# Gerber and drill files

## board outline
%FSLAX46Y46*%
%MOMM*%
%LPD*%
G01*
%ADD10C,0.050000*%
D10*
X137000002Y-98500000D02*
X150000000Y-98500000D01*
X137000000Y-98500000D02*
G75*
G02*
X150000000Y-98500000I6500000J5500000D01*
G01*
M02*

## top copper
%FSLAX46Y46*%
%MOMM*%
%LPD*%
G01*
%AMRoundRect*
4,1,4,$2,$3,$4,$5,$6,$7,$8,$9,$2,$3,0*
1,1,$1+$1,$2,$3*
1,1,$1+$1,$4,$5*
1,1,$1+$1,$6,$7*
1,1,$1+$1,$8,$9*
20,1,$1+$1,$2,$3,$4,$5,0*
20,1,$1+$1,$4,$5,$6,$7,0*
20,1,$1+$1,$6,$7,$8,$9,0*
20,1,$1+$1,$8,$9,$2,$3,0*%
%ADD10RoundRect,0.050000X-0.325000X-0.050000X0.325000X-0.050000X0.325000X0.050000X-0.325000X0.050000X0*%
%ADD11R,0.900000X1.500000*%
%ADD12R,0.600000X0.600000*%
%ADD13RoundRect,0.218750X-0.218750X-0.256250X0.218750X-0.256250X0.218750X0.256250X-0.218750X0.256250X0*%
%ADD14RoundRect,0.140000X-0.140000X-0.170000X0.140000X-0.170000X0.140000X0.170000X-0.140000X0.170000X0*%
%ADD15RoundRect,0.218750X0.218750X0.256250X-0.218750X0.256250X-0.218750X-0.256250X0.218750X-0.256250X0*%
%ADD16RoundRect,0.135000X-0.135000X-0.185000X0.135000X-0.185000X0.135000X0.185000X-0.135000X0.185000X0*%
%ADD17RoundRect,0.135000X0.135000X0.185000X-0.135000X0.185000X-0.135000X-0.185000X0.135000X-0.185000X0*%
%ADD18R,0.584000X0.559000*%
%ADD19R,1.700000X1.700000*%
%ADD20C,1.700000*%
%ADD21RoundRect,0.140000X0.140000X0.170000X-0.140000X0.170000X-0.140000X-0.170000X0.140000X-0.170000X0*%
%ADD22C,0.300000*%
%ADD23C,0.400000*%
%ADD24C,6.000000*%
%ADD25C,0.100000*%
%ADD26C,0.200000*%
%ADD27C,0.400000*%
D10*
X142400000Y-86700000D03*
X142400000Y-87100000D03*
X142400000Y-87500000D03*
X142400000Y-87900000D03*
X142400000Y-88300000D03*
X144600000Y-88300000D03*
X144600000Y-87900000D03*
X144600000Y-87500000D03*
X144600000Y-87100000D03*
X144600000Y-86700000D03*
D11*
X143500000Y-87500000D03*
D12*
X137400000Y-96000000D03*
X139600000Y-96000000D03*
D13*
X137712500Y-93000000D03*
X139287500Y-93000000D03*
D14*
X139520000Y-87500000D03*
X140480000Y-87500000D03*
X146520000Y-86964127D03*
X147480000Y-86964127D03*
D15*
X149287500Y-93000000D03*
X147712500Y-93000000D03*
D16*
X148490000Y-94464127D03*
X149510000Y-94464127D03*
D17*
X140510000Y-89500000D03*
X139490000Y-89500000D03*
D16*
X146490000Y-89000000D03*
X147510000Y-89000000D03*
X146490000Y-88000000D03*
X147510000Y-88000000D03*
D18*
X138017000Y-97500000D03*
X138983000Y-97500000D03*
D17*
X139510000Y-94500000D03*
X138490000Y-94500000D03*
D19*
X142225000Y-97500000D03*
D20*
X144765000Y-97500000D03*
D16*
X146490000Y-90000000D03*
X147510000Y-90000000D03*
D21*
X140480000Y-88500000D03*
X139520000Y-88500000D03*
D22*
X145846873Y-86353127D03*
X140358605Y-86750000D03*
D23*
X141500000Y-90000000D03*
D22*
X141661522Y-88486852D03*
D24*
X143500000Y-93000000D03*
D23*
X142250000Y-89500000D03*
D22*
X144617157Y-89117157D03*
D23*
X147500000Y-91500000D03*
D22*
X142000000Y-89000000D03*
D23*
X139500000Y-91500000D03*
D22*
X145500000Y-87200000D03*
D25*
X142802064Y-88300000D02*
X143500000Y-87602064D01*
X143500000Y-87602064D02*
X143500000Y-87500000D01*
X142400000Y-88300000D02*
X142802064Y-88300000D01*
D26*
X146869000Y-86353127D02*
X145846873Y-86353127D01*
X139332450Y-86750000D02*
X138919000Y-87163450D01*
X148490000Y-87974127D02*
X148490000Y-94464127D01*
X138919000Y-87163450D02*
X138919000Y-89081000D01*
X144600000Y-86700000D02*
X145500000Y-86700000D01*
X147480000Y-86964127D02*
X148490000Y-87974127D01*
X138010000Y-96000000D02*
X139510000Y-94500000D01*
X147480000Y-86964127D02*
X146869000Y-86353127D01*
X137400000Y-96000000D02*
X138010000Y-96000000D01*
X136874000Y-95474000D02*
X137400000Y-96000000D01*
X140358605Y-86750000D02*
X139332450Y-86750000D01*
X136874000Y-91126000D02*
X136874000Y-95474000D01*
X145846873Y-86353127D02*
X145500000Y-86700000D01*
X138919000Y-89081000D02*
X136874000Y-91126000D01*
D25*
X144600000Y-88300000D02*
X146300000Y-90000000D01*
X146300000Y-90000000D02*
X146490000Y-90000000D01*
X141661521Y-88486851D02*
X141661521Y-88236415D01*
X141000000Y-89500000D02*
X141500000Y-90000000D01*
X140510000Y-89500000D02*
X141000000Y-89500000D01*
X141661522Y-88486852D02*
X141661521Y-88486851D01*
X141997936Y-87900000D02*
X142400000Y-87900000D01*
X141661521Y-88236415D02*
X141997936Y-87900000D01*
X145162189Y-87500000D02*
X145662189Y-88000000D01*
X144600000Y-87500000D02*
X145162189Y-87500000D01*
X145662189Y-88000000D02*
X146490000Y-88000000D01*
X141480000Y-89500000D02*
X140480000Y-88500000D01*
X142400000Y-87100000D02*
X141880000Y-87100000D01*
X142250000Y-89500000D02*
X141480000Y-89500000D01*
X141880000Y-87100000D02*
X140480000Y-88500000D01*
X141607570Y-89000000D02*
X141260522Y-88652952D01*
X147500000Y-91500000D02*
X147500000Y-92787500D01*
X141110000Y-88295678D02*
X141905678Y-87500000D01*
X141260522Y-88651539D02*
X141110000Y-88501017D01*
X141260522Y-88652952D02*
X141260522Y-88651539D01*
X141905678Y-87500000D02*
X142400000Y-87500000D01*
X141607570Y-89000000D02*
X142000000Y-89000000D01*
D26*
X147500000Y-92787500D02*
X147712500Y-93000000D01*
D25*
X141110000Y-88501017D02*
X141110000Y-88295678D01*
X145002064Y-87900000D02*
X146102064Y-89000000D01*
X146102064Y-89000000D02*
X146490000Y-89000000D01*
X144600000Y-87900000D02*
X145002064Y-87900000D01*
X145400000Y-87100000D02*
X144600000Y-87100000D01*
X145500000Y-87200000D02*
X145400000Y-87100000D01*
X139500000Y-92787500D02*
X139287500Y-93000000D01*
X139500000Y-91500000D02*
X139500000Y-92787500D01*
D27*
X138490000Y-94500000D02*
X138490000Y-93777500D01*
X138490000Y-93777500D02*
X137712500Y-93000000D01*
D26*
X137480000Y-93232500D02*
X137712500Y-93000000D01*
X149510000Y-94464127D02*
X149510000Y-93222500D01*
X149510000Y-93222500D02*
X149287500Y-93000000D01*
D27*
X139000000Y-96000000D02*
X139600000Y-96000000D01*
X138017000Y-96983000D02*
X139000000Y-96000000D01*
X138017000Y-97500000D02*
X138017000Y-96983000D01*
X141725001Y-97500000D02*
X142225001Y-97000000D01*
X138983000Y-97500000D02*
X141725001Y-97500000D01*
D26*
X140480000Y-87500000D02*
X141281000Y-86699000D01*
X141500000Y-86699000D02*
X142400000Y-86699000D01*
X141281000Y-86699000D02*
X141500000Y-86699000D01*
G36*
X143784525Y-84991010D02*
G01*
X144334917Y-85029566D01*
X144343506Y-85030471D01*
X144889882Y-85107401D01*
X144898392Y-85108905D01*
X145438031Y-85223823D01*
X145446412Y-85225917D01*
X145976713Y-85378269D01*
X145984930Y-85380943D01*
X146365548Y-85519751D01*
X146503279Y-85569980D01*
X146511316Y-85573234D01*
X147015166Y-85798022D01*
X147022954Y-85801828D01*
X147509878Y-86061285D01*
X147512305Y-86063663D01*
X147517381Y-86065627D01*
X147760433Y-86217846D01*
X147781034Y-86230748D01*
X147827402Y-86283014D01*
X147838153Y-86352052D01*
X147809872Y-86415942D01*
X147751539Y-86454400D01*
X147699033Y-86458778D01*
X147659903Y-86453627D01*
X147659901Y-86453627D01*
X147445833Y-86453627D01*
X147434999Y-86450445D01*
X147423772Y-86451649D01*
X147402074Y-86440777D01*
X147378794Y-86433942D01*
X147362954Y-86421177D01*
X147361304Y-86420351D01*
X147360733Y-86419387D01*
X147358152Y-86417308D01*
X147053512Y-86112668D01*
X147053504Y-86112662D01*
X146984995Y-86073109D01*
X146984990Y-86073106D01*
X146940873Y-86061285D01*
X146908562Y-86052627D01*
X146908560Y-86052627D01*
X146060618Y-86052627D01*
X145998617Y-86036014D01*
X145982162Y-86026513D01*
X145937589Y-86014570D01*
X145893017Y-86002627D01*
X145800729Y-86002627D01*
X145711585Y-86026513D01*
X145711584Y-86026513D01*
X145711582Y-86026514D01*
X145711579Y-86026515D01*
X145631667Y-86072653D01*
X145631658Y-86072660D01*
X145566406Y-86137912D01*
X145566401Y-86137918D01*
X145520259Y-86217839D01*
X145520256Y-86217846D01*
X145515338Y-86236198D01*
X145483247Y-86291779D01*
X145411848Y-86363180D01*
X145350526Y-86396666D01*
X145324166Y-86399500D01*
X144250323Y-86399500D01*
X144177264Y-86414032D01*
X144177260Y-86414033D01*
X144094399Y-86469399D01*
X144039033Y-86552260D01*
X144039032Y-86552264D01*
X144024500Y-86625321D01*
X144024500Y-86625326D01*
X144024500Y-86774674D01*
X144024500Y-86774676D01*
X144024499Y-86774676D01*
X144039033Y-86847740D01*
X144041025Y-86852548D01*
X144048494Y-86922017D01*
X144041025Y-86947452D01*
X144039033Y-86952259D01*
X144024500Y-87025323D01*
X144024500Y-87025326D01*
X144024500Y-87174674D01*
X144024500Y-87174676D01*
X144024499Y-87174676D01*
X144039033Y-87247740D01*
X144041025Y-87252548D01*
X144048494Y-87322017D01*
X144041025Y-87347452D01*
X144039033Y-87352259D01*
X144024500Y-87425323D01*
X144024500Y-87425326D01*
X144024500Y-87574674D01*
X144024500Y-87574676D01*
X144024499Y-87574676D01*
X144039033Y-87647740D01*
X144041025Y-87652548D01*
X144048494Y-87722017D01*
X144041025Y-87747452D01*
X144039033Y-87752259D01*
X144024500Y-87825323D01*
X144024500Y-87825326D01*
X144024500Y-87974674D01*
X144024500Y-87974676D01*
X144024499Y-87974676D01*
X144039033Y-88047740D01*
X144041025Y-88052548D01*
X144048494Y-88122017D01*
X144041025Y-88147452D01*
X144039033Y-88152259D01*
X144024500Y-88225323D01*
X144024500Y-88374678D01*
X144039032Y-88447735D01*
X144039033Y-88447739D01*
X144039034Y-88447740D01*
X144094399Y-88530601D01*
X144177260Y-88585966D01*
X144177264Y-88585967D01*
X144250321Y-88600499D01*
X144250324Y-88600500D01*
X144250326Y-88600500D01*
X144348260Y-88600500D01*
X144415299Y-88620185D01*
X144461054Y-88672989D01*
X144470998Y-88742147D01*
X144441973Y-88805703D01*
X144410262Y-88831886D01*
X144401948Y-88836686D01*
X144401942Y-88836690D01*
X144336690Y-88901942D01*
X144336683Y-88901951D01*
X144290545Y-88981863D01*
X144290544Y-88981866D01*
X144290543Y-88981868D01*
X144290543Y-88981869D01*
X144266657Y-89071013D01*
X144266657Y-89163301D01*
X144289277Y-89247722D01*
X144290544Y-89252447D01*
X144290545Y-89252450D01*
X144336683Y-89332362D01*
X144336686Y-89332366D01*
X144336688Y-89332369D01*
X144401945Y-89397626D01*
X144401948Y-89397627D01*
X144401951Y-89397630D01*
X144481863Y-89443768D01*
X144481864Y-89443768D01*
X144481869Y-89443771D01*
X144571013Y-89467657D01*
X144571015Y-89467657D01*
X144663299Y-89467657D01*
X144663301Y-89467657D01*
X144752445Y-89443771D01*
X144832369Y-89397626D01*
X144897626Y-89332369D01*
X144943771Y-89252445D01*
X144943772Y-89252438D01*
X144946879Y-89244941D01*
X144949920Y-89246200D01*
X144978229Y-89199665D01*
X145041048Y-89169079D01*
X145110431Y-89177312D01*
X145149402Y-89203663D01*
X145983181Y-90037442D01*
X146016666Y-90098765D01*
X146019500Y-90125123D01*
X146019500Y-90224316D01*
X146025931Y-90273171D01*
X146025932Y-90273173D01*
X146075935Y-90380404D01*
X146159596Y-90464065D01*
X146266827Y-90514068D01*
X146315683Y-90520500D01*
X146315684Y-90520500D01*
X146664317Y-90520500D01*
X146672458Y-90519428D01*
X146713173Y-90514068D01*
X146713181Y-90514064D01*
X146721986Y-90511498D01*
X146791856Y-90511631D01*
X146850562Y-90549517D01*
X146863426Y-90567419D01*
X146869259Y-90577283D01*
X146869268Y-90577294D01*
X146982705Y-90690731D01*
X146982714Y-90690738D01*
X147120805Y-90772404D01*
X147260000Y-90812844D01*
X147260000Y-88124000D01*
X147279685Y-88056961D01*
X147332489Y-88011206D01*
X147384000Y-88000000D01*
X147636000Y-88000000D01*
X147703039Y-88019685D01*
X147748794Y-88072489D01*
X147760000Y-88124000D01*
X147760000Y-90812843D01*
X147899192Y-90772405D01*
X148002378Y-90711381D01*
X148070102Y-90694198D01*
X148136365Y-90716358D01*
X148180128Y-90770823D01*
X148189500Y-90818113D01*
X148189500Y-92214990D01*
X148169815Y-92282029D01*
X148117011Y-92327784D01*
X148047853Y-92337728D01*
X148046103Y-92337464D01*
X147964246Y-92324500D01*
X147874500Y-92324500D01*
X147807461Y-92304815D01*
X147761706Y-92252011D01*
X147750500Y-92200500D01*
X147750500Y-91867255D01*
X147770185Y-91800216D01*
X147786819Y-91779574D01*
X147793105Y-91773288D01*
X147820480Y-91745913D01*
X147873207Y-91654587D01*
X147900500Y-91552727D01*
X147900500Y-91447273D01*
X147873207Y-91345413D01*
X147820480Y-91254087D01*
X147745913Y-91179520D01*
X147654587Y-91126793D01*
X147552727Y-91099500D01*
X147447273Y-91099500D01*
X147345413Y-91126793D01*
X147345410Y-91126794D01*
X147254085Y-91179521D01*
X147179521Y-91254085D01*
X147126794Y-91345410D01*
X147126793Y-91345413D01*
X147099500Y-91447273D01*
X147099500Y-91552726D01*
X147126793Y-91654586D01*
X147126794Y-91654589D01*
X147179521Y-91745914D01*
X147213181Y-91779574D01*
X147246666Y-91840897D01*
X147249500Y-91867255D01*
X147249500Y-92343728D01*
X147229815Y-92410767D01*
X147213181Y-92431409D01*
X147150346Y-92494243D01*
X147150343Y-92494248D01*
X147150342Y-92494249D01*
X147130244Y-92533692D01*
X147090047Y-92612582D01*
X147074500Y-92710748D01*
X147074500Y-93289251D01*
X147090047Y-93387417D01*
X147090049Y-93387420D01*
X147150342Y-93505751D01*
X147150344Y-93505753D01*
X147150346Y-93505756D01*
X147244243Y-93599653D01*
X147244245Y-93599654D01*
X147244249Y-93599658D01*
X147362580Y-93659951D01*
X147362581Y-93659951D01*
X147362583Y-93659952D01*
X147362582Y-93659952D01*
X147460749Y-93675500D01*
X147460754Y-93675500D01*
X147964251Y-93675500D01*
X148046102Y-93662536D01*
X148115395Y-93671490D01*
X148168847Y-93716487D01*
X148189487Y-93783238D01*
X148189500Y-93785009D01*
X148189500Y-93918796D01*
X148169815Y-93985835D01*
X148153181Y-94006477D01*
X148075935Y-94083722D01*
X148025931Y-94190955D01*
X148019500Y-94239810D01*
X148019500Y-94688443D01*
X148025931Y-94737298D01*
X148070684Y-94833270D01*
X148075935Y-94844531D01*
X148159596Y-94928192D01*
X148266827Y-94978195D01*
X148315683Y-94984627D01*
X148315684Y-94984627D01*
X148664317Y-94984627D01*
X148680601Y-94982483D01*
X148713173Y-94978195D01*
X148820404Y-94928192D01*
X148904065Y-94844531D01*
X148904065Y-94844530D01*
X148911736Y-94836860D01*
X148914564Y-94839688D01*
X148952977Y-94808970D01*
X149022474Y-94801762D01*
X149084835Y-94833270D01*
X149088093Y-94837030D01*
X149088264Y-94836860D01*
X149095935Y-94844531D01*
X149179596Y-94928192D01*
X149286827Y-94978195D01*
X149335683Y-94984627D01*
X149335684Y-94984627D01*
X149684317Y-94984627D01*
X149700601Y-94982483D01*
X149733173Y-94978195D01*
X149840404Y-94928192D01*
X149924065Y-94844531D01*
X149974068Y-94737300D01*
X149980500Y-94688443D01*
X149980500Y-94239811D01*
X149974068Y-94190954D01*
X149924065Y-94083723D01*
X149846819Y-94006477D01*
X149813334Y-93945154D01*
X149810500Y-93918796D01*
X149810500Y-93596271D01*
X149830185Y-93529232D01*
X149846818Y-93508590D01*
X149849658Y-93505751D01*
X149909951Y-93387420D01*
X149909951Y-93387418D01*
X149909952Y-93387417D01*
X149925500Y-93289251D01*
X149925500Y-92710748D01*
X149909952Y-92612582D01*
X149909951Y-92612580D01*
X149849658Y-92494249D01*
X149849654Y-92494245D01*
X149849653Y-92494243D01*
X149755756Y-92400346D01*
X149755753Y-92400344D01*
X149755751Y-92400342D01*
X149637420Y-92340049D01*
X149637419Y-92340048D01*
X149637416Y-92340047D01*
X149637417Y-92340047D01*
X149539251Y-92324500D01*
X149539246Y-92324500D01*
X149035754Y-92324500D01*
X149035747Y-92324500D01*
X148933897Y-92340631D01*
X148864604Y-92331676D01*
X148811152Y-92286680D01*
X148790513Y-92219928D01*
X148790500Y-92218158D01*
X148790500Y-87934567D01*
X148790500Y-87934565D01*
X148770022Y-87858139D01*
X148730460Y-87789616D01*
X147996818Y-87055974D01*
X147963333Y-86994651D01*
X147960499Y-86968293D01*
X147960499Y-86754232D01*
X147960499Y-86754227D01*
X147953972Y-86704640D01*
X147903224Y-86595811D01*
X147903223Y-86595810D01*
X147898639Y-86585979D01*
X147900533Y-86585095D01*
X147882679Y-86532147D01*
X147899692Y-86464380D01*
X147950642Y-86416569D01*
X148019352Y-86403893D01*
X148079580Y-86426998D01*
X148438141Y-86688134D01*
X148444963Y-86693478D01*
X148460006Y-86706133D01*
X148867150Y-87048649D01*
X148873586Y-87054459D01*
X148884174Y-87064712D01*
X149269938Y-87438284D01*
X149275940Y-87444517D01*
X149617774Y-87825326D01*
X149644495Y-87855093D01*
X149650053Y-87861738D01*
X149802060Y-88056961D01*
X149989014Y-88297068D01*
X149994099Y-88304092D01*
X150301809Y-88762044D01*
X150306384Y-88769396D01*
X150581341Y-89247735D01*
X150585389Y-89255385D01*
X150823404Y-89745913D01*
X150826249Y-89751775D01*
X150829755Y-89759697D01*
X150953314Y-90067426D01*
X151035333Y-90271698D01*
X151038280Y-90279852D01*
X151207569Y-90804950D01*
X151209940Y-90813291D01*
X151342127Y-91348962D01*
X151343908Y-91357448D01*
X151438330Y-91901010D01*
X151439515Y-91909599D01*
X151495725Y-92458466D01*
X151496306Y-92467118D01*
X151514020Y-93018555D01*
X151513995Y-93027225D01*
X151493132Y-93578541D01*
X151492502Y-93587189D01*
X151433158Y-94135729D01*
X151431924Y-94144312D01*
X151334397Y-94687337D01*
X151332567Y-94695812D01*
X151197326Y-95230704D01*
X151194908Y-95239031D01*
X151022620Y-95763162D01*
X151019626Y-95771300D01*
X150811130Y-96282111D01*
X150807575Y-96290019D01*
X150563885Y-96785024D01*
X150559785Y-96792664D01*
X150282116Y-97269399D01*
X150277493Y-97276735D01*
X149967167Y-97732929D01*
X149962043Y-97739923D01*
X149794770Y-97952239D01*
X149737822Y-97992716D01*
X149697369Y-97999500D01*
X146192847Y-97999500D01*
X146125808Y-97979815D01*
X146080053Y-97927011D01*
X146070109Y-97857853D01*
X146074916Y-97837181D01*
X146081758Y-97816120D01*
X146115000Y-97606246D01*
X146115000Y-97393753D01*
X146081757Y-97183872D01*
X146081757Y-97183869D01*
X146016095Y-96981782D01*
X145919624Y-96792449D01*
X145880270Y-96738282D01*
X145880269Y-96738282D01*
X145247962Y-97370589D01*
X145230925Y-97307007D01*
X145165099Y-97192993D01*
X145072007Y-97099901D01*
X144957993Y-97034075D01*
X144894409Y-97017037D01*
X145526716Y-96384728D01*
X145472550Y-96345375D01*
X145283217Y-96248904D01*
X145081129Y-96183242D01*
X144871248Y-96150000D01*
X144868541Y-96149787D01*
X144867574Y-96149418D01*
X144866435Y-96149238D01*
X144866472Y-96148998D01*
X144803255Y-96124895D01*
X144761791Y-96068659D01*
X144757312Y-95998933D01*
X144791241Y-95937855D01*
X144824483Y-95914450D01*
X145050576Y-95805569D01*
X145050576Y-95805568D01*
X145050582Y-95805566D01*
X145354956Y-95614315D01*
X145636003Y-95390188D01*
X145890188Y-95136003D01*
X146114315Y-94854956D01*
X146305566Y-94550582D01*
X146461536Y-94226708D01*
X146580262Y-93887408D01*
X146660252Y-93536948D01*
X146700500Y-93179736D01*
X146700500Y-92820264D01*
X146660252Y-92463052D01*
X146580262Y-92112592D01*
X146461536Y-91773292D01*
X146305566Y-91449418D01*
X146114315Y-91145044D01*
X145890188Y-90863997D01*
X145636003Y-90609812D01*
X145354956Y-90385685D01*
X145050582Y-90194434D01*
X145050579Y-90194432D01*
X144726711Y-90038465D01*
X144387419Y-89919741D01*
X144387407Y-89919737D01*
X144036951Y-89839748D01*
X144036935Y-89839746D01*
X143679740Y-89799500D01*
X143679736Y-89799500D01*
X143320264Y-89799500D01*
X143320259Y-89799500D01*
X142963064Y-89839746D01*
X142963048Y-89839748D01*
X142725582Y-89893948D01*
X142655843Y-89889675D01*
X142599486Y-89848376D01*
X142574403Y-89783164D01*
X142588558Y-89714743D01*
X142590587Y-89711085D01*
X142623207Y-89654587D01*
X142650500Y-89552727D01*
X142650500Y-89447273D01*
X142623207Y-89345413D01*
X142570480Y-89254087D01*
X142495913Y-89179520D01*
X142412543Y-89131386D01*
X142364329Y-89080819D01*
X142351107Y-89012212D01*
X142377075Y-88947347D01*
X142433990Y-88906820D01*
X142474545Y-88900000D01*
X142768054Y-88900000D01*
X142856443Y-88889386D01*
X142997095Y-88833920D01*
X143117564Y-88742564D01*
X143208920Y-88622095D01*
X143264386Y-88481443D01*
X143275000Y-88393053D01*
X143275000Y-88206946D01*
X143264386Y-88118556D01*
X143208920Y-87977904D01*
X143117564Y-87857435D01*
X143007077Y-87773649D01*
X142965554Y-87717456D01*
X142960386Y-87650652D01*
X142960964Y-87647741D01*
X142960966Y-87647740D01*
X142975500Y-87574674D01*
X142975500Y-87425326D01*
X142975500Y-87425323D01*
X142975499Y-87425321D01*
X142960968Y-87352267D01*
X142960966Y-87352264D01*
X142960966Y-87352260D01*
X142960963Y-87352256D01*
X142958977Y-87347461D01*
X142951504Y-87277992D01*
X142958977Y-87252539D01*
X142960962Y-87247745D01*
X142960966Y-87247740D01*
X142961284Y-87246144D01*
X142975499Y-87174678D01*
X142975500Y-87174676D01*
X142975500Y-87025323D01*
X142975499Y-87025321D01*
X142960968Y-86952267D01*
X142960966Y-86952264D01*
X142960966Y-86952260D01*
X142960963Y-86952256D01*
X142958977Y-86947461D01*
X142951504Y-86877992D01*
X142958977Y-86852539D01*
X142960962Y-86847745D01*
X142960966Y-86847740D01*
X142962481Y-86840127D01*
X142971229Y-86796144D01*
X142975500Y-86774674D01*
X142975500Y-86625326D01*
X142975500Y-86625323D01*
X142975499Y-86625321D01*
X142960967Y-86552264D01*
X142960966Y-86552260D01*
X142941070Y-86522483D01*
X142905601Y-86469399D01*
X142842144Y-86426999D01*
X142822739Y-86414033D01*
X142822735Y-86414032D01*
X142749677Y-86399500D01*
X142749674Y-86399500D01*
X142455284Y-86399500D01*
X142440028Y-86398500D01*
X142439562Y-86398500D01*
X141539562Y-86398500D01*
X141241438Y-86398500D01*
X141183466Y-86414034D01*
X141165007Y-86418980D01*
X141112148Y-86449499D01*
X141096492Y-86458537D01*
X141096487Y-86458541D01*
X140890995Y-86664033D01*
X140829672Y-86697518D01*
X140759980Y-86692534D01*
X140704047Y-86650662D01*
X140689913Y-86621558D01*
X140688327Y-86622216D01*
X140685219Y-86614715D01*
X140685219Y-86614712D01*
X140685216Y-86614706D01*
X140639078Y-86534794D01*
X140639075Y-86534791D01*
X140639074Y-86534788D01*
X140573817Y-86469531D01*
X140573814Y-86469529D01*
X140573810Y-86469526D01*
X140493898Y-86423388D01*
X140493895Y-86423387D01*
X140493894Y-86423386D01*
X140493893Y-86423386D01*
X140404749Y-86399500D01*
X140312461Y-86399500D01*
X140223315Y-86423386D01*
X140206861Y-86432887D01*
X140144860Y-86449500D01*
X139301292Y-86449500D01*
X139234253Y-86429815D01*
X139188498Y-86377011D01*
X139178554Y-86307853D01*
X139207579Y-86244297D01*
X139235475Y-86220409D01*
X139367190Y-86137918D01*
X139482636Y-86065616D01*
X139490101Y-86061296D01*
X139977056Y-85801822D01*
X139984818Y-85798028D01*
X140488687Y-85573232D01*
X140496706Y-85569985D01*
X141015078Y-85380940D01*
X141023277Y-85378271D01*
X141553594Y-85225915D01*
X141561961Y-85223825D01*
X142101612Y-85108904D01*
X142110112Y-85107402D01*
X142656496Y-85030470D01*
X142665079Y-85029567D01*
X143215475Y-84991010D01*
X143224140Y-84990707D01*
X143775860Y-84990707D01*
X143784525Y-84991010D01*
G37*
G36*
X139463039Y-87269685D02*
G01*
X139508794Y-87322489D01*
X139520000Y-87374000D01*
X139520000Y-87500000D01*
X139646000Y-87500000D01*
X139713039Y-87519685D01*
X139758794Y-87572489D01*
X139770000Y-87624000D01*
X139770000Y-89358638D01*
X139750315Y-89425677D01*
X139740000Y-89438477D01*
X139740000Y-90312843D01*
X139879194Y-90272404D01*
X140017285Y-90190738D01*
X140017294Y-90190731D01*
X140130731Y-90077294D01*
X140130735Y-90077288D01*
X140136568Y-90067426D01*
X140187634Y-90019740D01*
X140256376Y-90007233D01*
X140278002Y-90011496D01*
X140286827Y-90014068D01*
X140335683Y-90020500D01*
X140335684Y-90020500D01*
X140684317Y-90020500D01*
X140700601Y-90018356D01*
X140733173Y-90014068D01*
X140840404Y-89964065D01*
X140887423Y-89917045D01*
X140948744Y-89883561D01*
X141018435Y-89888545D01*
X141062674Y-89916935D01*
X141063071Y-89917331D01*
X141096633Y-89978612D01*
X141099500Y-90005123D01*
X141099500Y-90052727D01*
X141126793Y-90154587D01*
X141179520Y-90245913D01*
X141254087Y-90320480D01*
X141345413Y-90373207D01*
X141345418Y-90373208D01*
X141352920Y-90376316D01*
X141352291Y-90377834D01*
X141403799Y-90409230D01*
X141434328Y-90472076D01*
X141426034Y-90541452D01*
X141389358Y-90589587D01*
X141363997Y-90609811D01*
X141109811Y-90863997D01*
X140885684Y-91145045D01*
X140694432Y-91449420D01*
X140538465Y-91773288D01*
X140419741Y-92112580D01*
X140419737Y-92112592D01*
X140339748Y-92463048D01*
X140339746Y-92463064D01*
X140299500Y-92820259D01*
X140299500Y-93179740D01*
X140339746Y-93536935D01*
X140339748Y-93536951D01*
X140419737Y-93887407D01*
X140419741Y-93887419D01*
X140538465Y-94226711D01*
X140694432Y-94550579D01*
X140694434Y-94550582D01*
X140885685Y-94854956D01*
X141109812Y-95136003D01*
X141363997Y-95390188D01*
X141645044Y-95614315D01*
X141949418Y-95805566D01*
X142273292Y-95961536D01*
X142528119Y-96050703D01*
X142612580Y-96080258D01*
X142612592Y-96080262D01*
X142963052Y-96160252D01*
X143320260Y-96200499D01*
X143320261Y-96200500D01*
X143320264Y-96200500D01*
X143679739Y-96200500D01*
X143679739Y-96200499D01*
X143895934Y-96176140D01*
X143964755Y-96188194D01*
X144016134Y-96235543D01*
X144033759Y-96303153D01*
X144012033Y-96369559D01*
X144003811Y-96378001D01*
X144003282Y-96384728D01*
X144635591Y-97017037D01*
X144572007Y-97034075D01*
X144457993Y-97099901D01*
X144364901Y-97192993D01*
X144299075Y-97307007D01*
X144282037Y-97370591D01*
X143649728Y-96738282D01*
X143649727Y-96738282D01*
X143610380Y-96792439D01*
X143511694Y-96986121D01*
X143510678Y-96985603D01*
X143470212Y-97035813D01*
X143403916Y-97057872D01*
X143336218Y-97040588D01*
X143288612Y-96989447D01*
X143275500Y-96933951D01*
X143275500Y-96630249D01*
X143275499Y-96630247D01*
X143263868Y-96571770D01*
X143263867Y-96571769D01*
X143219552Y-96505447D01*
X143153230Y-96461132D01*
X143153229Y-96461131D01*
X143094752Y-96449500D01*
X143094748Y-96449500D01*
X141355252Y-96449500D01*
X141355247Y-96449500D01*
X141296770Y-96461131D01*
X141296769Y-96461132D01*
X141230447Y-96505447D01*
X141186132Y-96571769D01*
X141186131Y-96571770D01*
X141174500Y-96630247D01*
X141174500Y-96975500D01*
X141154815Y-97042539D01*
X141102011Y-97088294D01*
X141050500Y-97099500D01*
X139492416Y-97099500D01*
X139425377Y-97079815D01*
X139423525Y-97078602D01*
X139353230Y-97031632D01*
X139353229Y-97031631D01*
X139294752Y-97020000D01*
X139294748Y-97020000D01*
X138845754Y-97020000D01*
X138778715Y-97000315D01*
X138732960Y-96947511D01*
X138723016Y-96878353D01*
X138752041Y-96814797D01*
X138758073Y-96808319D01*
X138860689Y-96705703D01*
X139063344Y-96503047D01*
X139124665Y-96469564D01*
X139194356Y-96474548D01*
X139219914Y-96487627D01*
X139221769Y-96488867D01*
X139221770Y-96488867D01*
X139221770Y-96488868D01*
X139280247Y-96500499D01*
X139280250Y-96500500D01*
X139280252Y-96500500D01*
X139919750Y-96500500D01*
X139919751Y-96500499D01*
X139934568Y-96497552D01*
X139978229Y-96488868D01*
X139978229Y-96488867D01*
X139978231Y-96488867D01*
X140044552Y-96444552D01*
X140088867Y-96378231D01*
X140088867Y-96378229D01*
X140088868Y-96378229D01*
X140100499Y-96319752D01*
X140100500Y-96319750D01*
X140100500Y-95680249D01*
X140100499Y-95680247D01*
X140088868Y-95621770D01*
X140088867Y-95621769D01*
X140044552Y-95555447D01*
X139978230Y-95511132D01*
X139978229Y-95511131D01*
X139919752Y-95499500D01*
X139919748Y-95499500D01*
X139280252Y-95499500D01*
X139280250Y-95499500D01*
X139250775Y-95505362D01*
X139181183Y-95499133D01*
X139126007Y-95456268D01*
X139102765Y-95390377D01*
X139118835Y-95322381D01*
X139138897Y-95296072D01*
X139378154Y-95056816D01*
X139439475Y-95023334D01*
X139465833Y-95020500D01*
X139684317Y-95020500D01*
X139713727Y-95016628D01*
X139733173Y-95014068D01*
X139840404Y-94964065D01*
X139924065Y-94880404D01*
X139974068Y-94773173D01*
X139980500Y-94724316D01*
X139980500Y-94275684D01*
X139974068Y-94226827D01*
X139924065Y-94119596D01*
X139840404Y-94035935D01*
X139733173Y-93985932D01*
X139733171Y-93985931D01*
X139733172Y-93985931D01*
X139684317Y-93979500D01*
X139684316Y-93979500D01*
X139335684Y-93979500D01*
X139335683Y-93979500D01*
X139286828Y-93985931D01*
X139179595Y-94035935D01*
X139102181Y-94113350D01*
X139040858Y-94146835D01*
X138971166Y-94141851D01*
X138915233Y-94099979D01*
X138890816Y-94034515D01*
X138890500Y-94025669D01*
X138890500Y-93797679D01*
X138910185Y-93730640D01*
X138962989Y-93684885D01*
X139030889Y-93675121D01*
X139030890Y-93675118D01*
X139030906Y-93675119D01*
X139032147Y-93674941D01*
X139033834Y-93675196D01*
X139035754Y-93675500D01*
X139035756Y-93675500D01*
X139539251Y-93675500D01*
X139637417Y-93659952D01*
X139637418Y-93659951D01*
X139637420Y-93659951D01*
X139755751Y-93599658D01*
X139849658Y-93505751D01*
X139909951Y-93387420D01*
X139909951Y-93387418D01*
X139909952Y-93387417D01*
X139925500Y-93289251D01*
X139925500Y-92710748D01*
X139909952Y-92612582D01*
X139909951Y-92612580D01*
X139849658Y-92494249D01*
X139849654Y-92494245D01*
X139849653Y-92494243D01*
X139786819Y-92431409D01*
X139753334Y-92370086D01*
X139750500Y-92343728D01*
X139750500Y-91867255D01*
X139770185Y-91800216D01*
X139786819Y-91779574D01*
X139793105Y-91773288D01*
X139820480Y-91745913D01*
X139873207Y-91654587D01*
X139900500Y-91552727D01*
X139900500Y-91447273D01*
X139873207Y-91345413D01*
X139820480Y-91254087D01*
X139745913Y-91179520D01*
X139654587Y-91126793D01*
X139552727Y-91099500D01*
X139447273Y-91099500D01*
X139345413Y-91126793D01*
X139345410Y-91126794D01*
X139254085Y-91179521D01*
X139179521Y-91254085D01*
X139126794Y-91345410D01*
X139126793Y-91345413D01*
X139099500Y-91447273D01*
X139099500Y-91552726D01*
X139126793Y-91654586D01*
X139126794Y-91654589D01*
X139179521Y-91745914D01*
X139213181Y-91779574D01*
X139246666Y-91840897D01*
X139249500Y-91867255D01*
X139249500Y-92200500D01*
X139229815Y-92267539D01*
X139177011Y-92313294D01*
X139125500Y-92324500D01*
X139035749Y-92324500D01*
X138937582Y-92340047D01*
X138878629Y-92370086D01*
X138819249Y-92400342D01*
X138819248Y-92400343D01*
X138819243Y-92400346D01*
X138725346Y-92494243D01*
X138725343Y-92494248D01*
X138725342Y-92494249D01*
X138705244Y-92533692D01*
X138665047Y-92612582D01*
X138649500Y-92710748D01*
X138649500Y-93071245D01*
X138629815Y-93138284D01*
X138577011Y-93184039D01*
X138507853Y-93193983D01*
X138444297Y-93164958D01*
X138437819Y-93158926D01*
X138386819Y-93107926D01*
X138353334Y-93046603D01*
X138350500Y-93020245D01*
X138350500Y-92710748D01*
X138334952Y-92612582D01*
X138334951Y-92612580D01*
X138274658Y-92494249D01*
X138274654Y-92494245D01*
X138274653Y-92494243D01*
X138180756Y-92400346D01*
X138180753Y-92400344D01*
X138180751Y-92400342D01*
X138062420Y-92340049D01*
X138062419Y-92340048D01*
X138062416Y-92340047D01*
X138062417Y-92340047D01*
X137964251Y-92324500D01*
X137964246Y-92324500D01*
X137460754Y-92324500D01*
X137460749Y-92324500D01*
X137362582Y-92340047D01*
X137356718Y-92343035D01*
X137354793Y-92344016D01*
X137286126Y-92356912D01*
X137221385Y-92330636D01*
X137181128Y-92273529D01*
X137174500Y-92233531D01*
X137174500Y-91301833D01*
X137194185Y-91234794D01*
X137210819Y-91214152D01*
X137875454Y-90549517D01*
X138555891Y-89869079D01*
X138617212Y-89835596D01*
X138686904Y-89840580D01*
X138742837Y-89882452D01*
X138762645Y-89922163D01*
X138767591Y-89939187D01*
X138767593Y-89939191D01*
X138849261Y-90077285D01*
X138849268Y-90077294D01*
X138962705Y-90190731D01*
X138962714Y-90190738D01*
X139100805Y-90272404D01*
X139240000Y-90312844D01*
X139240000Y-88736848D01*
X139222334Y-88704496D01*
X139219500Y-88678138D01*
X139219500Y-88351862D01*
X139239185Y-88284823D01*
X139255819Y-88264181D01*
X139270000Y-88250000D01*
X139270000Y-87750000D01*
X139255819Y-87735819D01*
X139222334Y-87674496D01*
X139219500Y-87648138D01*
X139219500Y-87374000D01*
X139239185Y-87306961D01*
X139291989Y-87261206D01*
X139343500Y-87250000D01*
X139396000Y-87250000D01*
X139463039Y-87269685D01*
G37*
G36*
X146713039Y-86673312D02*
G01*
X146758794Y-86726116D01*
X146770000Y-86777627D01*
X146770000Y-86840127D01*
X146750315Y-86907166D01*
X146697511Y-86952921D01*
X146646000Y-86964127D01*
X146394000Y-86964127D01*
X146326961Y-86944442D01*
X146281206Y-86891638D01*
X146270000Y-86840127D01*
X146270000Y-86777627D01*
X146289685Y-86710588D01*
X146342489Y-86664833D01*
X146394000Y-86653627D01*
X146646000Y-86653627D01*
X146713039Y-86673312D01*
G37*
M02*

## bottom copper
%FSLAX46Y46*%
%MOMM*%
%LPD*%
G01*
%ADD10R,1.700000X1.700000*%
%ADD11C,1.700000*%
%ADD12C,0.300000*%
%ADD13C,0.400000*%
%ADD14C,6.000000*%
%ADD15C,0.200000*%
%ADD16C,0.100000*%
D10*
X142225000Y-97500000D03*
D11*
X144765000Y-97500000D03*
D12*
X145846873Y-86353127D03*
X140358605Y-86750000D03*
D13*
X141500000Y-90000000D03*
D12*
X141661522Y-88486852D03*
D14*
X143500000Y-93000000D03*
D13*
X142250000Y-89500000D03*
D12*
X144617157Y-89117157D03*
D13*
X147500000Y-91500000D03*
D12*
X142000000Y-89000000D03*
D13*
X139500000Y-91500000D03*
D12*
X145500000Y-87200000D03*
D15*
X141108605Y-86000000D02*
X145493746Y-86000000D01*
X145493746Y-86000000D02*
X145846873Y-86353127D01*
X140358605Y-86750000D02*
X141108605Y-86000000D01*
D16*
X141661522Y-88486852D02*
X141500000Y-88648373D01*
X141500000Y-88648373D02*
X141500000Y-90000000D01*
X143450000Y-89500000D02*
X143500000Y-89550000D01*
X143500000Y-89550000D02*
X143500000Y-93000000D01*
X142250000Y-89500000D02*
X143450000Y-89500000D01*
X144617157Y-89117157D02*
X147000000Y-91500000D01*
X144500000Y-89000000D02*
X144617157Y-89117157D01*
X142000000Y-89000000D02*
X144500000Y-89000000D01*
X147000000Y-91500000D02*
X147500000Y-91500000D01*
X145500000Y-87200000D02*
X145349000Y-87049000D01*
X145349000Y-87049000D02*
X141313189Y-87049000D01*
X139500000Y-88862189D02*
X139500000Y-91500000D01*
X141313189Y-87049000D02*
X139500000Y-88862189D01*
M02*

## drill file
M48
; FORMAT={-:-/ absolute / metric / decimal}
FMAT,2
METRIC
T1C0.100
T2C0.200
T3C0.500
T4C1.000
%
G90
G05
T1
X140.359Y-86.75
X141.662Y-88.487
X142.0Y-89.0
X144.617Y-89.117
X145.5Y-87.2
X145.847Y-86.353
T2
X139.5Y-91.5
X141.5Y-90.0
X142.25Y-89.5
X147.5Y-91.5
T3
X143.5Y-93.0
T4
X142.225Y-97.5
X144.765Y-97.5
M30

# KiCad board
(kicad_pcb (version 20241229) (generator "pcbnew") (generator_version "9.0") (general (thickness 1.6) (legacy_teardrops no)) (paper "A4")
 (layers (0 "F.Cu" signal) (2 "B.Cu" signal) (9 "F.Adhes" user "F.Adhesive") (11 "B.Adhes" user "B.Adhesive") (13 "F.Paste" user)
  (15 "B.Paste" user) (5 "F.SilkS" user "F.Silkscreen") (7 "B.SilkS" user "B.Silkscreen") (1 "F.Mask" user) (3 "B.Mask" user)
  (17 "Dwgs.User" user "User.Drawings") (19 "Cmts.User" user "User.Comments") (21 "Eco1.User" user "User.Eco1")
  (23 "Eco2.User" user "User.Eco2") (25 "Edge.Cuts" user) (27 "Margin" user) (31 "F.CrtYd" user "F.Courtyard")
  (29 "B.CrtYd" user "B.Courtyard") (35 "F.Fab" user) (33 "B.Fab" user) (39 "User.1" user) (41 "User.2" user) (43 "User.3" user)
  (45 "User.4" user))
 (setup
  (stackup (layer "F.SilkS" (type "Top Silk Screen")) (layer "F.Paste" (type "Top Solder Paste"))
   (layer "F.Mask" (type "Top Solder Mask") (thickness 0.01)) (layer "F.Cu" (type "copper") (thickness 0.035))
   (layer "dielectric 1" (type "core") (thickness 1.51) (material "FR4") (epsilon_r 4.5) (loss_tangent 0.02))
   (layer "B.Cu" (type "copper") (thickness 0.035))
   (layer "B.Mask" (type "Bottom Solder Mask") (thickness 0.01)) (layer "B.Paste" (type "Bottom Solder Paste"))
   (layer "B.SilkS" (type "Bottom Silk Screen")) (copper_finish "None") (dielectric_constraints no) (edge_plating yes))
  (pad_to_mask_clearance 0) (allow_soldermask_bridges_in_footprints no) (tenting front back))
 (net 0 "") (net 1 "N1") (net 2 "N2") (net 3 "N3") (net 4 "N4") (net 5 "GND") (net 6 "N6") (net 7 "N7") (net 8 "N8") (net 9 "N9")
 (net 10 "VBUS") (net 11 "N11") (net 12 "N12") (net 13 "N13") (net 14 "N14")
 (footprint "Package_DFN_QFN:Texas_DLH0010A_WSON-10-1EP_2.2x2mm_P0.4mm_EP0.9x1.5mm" (layer "F.Cu") (at 143.5 87.5)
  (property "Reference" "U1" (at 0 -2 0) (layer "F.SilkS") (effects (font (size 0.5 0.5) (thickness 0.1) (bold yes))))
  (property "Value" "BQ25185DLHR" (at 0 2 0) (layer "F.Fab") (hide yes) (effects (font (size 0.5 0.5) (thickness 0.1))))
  (pad "" smd roundrect (at 0 0) (size 0.84 1.41) (layers "F.Paste") (roundrect_rratio 0.25))
  (pad "1" smd roundrect (at -1.1 -0.8) (size 0.75 0.2) (layers "F.Cu" "F.Mask" "F.Paste") (roundrect_rratio 0.25) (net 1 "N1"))
  (pad "2" smd roundrect (at -1.1 -0.4) (size 0.75 0.2) (layers "F.Cu" "F.Mask" "F.Paste") (roundrect_rratio 0.25) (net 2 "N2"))
  (pad "3" smd roundrect (at -1.1 0) (size 0.75 0.2) (layers "F.Cu" "F.Mask" "F.Paste") (roundrect_rratio 0.25) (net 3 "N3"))
  (pad "4" smd roundrect (at -1.1 0.4) (size 0.75 0.2) (layers "F.Cu" "F.Mask" "F.Paste") (roundrect_rratio 0.25) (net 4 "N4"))
  (pad "5" smd roundrect (at -1.1 0.8) (size 0.75 0.2) (layers "F.Cu" "F.Mask" "F.Paste") (roundrect_rratio 0.25) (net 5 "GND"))
  (pad "6" smd roundrect (at 1.1 0.8) (size 0.75 0.2) (layers "F.Cu" "F.Mask" "F.Paste") (roundrect_rratio 0.25) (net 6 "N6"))
  (pad "7" smd roundrect (at 1.1 0.4) (size 0.75 0.2) (layers "F.Cu" "F.Mask" "F.Paste") (roundrect_rratio 0.25) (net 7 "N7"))
  (pad "8" smd roundrect (at 1.1 0) (size 0.75 0.2) (layers "F.Cu" "F.Mask" "F.Paste") (roundrect_rratio 0.25) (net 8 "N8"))
  (pad "9" smd roundrect (at 1.1 -0.4) (size 0.75 0.2) (layers "F.Cu" "F.Mask" "F.Paste") (roundrect_rratio 0.25) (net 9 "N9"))
  (pad "10" smd roundrect (at 1.1 -0.8) (size 0.75 0.2) (layers "F.Cu" "F.Mask" "F.Paste") (roundrect_rratio 0.25) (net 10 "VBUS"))
  (pad "11" smd rect (at 0 0) (size 0.9 1.5) (layers "F.Cu" "F.Mask") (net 5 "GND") (zone_connect 2)))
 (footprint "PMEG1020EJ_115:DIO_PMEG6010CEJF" (layer "F.Cu") (at 138.5 96)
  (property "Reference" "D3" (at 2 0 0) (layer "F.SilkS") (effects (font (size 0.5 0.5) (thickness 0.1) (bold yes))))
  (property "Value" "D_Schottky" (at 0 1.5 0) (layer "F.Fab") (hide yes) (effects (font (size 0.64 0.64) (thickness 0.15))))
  (pad "1" smd rect (at -1.1 0) (size 0.6 0.6) (layers "F.Cu" "F.Mask") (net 10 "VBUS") (solder_mask_margin 0.102))
  (pad "2" smd rect (at 1.1 0) (size 0.6 0.6) (layers "F.Cu" "F.Mask") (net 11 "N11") (solder_mask_margin 0.102)))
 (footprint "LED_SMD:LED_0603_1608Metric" (layer "F.Cu") (at 138.5 93)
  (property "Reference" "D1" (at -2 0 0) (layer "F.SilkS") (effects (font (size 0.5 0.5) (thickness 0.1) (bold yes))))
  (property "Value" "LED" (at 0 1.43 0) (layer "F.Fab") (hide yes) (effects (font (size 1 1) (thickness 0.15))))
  (pad "1" smd roundrect (at -0.7875 0) (size 0.875 0.95) (layers "F.Cu" "F.Mask" "F.Paste") (roundrect_rratio 0.25) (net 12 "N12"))
  (pad "2" smd roundrect (at 0.7875 0) (size 0.875 0.95) (layers "F.Cu" "F.Mask" "F.Paste") (roundrect_rratio 0.25) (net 9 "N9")))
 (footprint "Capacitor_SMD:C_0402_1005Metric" (layer "F.Cu") (at 140 87.5)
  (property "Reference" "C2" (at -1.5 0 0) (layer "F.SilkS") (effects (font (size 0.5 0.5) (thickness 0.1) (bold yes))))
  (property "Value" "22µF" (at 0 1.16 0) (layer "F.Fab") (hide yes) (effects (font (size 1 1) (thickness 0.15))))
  (pad "1" smd roundrect (at -0.48 0) (size 0.56 0.62) (layers "F.Cu" "F.Mask" "F.Paste") (roundrect_rratio 0.25) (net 5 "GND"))
  (pad "2" smd roundrect (at 0.48 0) (size 0.56 0.62) (layers "F.Cu" "F.Mask" "F.Paste") (roundrect_rratio 0.25) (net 1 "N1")))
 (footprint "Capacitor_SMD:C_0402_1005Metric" (layer "F.Cu") (at 147 86.964127)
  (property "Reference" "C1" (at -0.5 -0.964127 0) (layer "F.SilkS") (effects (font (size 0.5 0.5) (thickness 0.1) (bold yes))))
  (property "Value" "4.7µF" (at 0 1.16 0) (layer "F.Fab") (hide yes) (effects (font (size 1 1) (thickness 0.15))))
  (pad "1" smd roundrect (at -0.48 0) (size 0.56 0.62) (layers "F.Cu" "F.Mask" "F.Paste") (roundrect_rratio 0.25) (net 5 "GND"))
  (pad "2" smd roundrect (at 0.48 0) (size 0.56 0.62) (layers "F.Cu" "F.Mask" "F.Paste") (roundrect_rratio 0.25) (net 10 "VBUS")))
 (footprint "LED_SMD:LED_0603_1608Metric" (layer "F.Cu") (at 148.5 93 180)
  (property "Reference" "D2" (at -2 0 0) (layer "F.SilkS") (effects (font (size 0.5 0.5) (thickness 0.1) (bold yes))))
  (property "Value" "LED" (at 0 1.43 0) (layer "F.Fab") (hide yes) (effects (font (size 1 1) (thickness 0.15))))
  (pad "1" smd roundrect (at -0.7875 0 180) (size 0.875 0.95) (layers "F.Cu" "F.Mask" "F.Paste") (roundrect_rratio 0.25) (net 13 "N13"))
  (pad "2" smd roundrect (at 0.7875 0 180) (size 0.875 0.95) (layers "F.Cu" "F.Mask" "F.Paste") (roundrect_rratio 0.25) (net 3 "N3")))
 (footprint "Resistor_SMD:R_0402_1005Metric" (layer "F.Cu") (at 149 94.464127)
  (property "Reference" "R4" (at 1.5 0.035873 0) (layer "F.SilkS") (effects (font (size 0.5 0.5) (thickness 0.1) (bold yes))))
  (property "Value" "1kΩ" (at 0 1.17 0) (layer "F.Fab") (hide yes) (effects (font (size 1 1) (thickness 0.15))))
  (pad "1" smd roundrect (at -0.51 0) (size 0.54 0.64) (layers "F.Cu" "F.Mask" "F.Paste") (roundrect_rratio 0.25) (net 10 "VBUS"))
  (pad "2" smd roundrect (at 0.51 0) (size 0.54 0.64) (layers "F.Cu" "F.Mask" "F.Paste") (roundrect_rratio 0.25) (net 13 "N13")))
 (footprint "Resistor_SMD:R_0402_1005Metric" (layer "F.Cu") (at 140 89.5 180)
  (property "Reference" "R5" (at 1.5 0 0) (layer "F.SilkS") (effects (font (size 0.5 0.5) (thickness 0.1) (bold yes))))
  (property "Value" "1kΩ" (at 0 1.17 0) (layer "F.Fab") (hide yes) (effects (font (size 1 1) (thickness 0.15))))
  (pad "1" smd roundrect (at -0.51 0 180) (size 0.54 0.64) (layers "F.Cu" "F.Mask" "F.Paste") (roundrect_rratio 0.25) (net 4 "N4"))
  (pad "2" smd roundrect (at 0.51 0 180) (size 0.54 0.64) (layers "F.Cu" "F.Mask" "F.Paste") (roundrect_rratio 0.25) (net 5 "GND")))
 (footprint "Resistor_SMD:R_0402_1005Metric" (layer "F.Cu") (at 147 89)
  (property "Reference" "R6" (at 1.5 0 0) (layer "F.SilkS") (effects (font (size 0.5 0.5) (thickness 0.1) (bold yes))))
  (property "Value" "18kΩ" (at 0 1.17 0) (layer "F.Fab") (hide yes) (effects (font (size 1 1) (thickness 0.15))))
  (pad "1" smd roundrect (at -0.51 0) (size 0.54 0.64) (layers "F.Cu" "F.Mask" "F.Paste") (roundrect_rratio 0.25) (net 7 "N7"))
  (pad "2" smd roundrect (at 0.51 0) (size 0.54 0.64) (layers "F.Cu" "F.Mask" "F.Paste") (roundrect_rratio 0.25) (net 5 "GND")))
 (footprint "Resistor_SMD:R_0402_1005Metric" (layer "F.Cu") (at 147 88)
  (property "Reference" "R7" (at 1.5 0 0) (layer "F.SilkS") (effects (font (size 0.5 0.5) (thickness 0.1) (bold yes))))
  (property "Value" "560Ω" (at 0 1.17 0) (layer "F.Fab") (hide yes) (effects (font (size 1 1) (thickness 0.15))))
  (pad "1" smd roundrect (at -0.51 0) (size 0.54 0.64) (layers "F.Cu" "F.Mask" "F.Paste") (roundrect_rratio 0.25) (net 8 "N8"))
  (pad "2" smd roundrect (at 0.51 0) (size 0.54 0.64) (layers "F.Cu" "F.Mask" "F.Paste") (roundrect_rratio 0.25) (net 5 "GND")))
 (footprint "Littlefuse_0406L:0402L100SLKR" (layer "F.Cu") (at 138.5 97.5)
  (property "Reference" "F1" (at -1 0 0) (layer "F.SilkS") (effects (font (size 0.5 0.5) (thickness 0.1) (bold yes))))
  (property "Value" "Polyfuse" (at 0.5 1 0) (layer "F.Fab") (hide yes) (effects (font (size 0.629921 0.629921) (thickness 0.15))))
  (pad "1" smd rect (at -0.483 0) (size 0.584 0.559) (layers "F.Cu" "F.Mask" "F.Paste") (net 11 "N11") (solder_mask_margin 0.102))
  (pad "2" smd rect (at 0.483 0) (size 0.584 0.559) (layers "F.Cu" "F.Mask" "F.Paste") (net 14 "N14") (solder_mask_margin 0.102)))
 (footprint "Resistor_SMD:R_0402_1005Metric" (layer "F.Cu") (at 139 94.5 180)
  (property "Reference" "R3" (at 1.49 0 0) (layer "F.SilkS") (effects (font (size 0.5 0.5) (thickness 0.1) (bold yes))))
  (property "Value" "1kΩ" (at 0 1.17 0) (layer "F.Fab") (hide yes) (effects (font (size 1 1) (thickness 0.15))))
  (pad "1" smd roundrect (at -0.51 0 180) (size 0.54 0.64) (layers "F.Cu" "F.Mask" "F.Paste") (roundrect_rratio 0.25) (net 10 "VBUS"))
  (pad "2" smd roundrect (at 0.51 0 180) (size 0.54 0.64) (layers "F.Cu" "F.Mask" "F.Paste") (roundrect_rratio 0.25) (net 12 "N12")))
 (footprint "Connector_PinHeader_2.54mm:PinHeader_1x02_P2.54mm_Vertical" (layer "F.Cu") (at 142.225 97.5 90)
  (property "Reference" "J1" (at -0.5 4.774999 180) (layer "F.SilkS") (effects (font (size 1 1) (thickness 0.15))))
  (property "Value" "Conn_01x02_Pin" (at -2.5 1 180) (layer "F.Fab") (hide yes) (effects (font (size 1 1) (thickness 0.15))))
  (pad "1" thru_hole rect (at 0 0 90) (size 1.7 1.7) (drill 1) (layers "*.Cu" "*.Mask") (remove_unused_layers no) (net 14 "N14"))
  (pad "2" thru_hole circle (at 0 2.54 90) (size 1.7 1.7) (drill 1) (layers "*.Cu" "*.Mask") (remove_unused_layers no) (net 5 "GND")))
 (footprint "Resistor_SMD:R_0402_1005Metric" (layer "F.Cu") (at 147 90)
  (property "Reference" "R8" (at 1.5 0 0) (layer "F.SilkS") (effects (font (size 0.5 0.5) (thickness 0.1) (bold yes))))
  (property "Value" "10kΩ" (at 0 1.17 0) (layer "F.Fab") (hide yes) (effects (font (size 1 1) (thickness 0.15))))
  (pad "1" smd roundrect (at -0.51 0) (size 0.54 0.64) (layers "F.Cu" "F.Mask" "F.Paste") (roundrect_rratio 0.25) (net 6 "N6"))
  (pad "2" smd roundrect (at 0.51 0) (size 0.54 0.64) (layers "F.Cu" "F.Mask" "F.Paste") (roundrect_rratio 0.25) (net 5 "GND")))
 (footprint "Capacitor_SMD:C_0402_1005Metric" (layer "F.Cu") (at 140 88.5 180)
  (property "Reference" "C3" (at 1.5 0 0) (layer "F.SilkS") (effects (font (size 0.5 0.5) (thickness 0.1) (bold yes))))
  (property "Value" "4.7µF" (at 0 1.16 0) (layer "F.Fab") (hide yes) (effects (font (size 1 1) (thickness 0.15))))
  (pad "1" smd roundrect (at -0.48 0 180) (size 0.56 0.62) (layers "F.Cu" "F.Mask" "F.Paste") (roundrect_rratio 0.25) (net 2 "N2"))
  (pad "2" smd roundrect (at 0.48 0 180) (size 0.56 0.62) (layers "F.Cu" "F.Mask" "F.Paste") (roundrect_rratio 0.25) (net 5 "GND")))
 (gr_line (start 137.000002 98.5) (end 150 98.5) (stroke (width 0.05) (type default)) (layer "Edge.Cuts"))
 (gr_arc (start 137 98.5) (mid 143.5 84.485307) (end 150 98.5) (stroke (width 0.05) (type default)) (layer "Edge.Cuts"))
 (segment (start 142.802064 88.3) (end 143.5 87.602064) (width 0.1) (layer "F.Cu") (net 5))
 (segment (start 143.5 87.602064) (end 143.5 87.5) (width 0.1) (layer "F.Cu") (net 5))
 (segment (start 142.4 88.3) (end 142.802064 88.3) (width 0.1) (layer "F.Cu") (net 5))
 (segment (start 146.869 86.353127) (end 145.846873 86.353127) (width 0.2) (layer "F.Cu") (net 10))
 (segment (start 139.33245 86.75) (end 138.919 87.16345) (width 0.2) (layer "F.Cu") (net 10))
 (segment (start 148.49 87.974127) (end 148.49 94.464127) (width 0.2) (layer "F.Cu") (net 10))
 (segment (start 138.919 87.16345) (end 138.919 89.081) (width 0.2) (layer "F.Cu") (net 10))
 (segment (start 144.6 86.7) (end 145.5 86.7) (width 0.2) (layer "F.Cu") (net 10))
 (segment (start 147.48 86.964127) (end 148.49 87.974127) (width 0.2) (layer "F.Cu") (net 10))
 (segment (start 138.01 96) (end 139.51 94.5) (width 0.2) (layer "F.Cu") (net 10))
 (segment (start 147.48 86.964127) (end 146.869 86.353127) (width 0.2) (layer "F.Cu") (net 10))
 (segment (start 137.4 96) (end 138.01 96) (width 0.2) (layer "F.Cu") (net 10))
 (segment (start 136.874 95.474) (end 137.4 96) (width 0.2) (layer "F.Cu") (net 10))
 (segment (start 140.358605 86.75) (end 139.33245 86.75) (width 0.2) (layer "F.Cu") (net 10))
 (segment (start 136.874 91.126) (end 136.874 95.474) (width 0.2) (layer "F.Cu") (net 10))
 (segment (start 145.846873 86.353127) (end 145.5 86.7) (width 0.2) (layer "F.Cu") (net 10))
 (segment (start 138.919 89.081) (end 136.874 91.126) (width 0.2) (layer "F.Cu") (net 10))
 (via (at 145.846873 86.353127) (size 0.3) (drill 0.1) (layers "F.Cu" "B.Cu") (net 10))
 (via (at 140.358605 86.75) (size 0.3) (drill 0.1) (layers "F.Cu" "B.Cu") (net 10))
 (segment (start 141.108605 86) (end 145.493746 86) (width 0.2) (layer "B.Cu") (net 10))
 (segment (start 145.493746 86) (end 145.846873 86.353127) (width 0.2) (layer "B.Cu") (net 10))
 (segment (start 140.358605 86.75) (end 141.108605 86) (width 0.2) (layer "B.Cu") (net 10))
 (segment (start 144.6 88.3) (end 146.3 90) (width 0.1) (layer "F.Cu") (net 6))
 (segment (start 146.3 90) (end 146.49 90) (width 0.1) (layer "F.Cu") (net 6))
 (segment (start 141.661521 88.486851) (end 141.661521 88.236415) (width 0.1) (layer "F.Cu") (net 4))
 (segment (start 141 89.5) (end 141.5 90) (width 0.1) (layer "F.Cu") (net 4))
 (segment (start 140.51 89.5) (end 141 89.5) (width 0.1) (layer "F.Cu") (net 4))
 (segment (start 141.661522 88.486852) (end 141.661521 88.486851) (width 0.1) (layer "F.Cu") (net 4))
 (segment (start 141.997936 87.9) (end 142.4 87.9) (width 0.1) (layer "F.Cu") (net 4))
 (segment (start 141.661521 88.236415) (end 141.997936 87.9) (width 0.1) (layer "F.Cu") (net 4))
 (via (at 141.5 90) (size 0.4) (drill 0.2) (layers "F.Cu" "B.Cu") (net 4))
 (via (at 141.661522 88.486852) (size 0.3) (drill 0.1) (layers "F.Cu" "B.Cu") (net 4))
 (segment (start 141.661522 88.486852) (end 141.5 88.648373) (width 0.1) (layer "B.Cu") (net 4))
 (segment (start 141.5 88.648373) (end 141.5 90) (width 0.1) (layer "B.Cu") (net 4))
 (segment (start 145.162189 87.5) (end 145.662189 88) (width 0.1) (layer "F.Cu") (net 8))
 (segment (start 144.6 87.5) (end 145.162189 87.5) (width 0.1) (layer "F.Cu") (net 8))
 (segment (start 145.662189 88) (end 146.49 88) (width 0.1) (layer "F.Cu") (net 8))
 (segment (start 141.48 89.5) (end 140.48 88.5) (width 0.1) (layer "F.Cu") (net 2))
 (segment (start 142.4 87.1) (end 141.88 87.1) (width 0.1) (layer "F.Cu") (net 2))
 (segment (start 142.25 89.5) (end 141.48 89.5) (width 0.1) (layer "F.Cu") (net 2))
 (segment (start 141.88 87.1) (end 140.48 88.5) (width 0.1) (layer "F.Cu") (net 2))
 (via blind (at 143.5 93) (size 6) (drill 0.5) (layers "F.Cu" "B.Cu") (tenting none) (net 2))
 (via (at 142.25 89.5) (size 0.4) (drill 0.2) (layers "F.Cu" "B.Cu") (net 2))
 (segment (start 143.45 89.5) (end 143.5 89.55) (width 0.1) (layer "B.Cu") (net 2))
 (segment (start 143.5 89.55) (end 143.5 93) (width 0.1) (layer "B.Cu") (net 2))
 (segment (start 142.25 89.5) (end 143.45 89.5) (width 0.1) (layer "B.Cu") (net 2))
 (segment (start 141.60757 89) (end 141.260522 88.652952) (width 0.1) (layer "F.Cu") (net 3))
 (segment (start 147.5 91.5) (end 147.5 92.7875) (width 0.1) (layer "F.Cu") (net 3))
 (segment (start 141.11 88.295678) (end 141.905678 87.5) (width 0.1) (layer "F.Cu") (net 3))
 (segment (start 141.260522 88.651539) (end 141.11 88.501017) (width 0.1) (layer "F.Cu") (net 3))
 (segment (start 141.260522 88.652952) (end 141.260522 88.651539) (width 0.1) (layer "F.Cu") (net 3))
 (segment (start 141.905678 87.5) (end 142.4 87.5) (width 0.1) (layer "F.Cu") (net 3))
 (segment (start 141.60757 89) (end 142 89) (width 0.1) (layer "F.Cu") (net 3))
 (segment (start 147.5 92.7875) (end 147.7125 93) (width 0.2) (layer "F.Cu") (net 3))
 (segment (start 141.11 88.501017) (end 141.11 88.295678) (width 0.1) (layer "F.Cu") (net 3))
 (via (at 144.617157 89.117157) (size 0.3) (drill 0.1) (layers "F.Cu" "B.Cu") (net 3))
 (via (at 147.5 91.5) (size 0.4) (drill 0.2) (layers "F.Cu" "B.Cu") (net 3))
 (via (at 142 89) (size 0.3) (drill 0.1) (layers "F.Cu" "B.Cu") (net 3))
 (segment (start 144.617157 89.117157) (end 147 91.5) (width 0.1) (layer "B.Cu") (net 3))
 (segment (start 144.5 89) (end 144.617157 89.117157) (width 0.1) (layer "B.Cu") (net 3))
 (segment (start 142 89) (end 144.5 89) (width 0.1) (layer "B.Cu") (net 3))
 (segment (start 147 91.5) (end 147.5 91.5) (width 0.1) (layer "B.Cu") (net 3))
 (segment (start 145.002064 87.9) (end 146.102064 89) (width 0.1) (layer "F.Cu") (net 7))
 (segment (start 146.102064 89) (end 146.49 89) (width 0.1) (layer "F.Cu") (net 7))
 (segment (start 144.6 87.9) (end 145.002064 87.9) (width 0.1) (layer "F.Cu") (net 7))
 (segment (start 145.4 87.1) (end 144.6 87.1) (width 0.1) (layer "F.Cu") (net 9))
 (segment (start 145.5 87.2) (end 145.4 87.1) (width 0.1) (layer "F.Cu") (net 9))
 (segment (start 139.5 92.7875) (end 139.2875 93) (width 0.1) (layer "F.Cu") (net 9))
 (segment (start 139.5 91.5) (end 139.5 92.7875) (width 0.1) (layer "F.Cu") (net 9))
 (via (at 139.5 91.5) (size 0.4) (drill 0.2) (layers "F.Cu" "B.Cu") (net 9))
 (via (at 145.5 87.2) (size 0.3) (drill 0.1) (layers "F.Cu" "B.Cu") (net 9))
 (segment (start 145.5 87.2) (end 145.349 87.049) (width 0.1) (layer "B.Cu") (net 9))
 (segment (start 145.349 87.049) (end 141.313189 87.049) (width 0.1) (layer "B.Cu") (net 9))
 (segment (start 139.5 88.862189) (end 139.5 91.5) (width 0.1) (layer "B.Cu") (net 9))
 (segment (start 141.313189 87.049) (end 139.5 88.862189) (width 0.1) (layer "B.Cu") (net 9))
 (segment (start 138.49 94.5) (end 138.49 93.7775) (width 0.4) (layer "F.Cu") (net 12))
 (segment (start 138.49 93.7775) (end 137.7125 93) (width 0.4) (layer "F.Cu") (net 12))
 (segment (start 137.48 93.2325) (end 137.7125 93) (width 0.2) (layer "F.Cu") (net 12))
 (segment (start 149.51 94.464127) (end 149.51 93.2225) (width 0.2) (layer "F.Cu") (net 13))
 (segment (start 149.51 93.2225) (end 149.2875 93) (width 0.2) (layer "F.Cu") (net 13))
 (segment (start 139 96) (end 139.6 96) (width 0.4) (layer "F.Cu") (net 11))
 (segment (start 138.017 96.983) (end 139 96) (width 0.4) (layer "F.Cu") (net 11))
 (segment (start 138.017 97.5) (end 138.017 96.983) (width 0.4) (layer "F.Cu") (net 11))
 (segment (start 141.725001 97.5) (end 142.225001 97) (width 0.4) (layer "F.Cu") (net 14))
 (segment (start 138.983 97.5) (end 141.725001 97.5) (width 0.4) (layer "F.Cu") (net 14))
 (segment (start 140.48 87.5) (end 141.281 86.699) (width 0.2) (layer "F.Cu") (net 1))
 (segment (start 141.5 86.699) (end 142.4 86.699) (width 0.2) (layer "F.Cu") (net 1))
 (segment (start 141.281 86.699) (end 141.5 86.699) (width 0.2) (layer "F.Cu") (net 1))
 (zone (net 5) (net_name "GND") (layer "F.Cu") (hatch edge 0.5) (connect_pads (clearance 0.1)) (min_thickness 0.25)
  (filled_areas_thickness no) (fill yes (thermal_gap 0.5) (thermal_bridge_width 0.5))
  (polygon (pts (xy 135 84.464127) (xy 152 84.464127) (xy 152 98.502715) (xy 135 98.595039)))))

